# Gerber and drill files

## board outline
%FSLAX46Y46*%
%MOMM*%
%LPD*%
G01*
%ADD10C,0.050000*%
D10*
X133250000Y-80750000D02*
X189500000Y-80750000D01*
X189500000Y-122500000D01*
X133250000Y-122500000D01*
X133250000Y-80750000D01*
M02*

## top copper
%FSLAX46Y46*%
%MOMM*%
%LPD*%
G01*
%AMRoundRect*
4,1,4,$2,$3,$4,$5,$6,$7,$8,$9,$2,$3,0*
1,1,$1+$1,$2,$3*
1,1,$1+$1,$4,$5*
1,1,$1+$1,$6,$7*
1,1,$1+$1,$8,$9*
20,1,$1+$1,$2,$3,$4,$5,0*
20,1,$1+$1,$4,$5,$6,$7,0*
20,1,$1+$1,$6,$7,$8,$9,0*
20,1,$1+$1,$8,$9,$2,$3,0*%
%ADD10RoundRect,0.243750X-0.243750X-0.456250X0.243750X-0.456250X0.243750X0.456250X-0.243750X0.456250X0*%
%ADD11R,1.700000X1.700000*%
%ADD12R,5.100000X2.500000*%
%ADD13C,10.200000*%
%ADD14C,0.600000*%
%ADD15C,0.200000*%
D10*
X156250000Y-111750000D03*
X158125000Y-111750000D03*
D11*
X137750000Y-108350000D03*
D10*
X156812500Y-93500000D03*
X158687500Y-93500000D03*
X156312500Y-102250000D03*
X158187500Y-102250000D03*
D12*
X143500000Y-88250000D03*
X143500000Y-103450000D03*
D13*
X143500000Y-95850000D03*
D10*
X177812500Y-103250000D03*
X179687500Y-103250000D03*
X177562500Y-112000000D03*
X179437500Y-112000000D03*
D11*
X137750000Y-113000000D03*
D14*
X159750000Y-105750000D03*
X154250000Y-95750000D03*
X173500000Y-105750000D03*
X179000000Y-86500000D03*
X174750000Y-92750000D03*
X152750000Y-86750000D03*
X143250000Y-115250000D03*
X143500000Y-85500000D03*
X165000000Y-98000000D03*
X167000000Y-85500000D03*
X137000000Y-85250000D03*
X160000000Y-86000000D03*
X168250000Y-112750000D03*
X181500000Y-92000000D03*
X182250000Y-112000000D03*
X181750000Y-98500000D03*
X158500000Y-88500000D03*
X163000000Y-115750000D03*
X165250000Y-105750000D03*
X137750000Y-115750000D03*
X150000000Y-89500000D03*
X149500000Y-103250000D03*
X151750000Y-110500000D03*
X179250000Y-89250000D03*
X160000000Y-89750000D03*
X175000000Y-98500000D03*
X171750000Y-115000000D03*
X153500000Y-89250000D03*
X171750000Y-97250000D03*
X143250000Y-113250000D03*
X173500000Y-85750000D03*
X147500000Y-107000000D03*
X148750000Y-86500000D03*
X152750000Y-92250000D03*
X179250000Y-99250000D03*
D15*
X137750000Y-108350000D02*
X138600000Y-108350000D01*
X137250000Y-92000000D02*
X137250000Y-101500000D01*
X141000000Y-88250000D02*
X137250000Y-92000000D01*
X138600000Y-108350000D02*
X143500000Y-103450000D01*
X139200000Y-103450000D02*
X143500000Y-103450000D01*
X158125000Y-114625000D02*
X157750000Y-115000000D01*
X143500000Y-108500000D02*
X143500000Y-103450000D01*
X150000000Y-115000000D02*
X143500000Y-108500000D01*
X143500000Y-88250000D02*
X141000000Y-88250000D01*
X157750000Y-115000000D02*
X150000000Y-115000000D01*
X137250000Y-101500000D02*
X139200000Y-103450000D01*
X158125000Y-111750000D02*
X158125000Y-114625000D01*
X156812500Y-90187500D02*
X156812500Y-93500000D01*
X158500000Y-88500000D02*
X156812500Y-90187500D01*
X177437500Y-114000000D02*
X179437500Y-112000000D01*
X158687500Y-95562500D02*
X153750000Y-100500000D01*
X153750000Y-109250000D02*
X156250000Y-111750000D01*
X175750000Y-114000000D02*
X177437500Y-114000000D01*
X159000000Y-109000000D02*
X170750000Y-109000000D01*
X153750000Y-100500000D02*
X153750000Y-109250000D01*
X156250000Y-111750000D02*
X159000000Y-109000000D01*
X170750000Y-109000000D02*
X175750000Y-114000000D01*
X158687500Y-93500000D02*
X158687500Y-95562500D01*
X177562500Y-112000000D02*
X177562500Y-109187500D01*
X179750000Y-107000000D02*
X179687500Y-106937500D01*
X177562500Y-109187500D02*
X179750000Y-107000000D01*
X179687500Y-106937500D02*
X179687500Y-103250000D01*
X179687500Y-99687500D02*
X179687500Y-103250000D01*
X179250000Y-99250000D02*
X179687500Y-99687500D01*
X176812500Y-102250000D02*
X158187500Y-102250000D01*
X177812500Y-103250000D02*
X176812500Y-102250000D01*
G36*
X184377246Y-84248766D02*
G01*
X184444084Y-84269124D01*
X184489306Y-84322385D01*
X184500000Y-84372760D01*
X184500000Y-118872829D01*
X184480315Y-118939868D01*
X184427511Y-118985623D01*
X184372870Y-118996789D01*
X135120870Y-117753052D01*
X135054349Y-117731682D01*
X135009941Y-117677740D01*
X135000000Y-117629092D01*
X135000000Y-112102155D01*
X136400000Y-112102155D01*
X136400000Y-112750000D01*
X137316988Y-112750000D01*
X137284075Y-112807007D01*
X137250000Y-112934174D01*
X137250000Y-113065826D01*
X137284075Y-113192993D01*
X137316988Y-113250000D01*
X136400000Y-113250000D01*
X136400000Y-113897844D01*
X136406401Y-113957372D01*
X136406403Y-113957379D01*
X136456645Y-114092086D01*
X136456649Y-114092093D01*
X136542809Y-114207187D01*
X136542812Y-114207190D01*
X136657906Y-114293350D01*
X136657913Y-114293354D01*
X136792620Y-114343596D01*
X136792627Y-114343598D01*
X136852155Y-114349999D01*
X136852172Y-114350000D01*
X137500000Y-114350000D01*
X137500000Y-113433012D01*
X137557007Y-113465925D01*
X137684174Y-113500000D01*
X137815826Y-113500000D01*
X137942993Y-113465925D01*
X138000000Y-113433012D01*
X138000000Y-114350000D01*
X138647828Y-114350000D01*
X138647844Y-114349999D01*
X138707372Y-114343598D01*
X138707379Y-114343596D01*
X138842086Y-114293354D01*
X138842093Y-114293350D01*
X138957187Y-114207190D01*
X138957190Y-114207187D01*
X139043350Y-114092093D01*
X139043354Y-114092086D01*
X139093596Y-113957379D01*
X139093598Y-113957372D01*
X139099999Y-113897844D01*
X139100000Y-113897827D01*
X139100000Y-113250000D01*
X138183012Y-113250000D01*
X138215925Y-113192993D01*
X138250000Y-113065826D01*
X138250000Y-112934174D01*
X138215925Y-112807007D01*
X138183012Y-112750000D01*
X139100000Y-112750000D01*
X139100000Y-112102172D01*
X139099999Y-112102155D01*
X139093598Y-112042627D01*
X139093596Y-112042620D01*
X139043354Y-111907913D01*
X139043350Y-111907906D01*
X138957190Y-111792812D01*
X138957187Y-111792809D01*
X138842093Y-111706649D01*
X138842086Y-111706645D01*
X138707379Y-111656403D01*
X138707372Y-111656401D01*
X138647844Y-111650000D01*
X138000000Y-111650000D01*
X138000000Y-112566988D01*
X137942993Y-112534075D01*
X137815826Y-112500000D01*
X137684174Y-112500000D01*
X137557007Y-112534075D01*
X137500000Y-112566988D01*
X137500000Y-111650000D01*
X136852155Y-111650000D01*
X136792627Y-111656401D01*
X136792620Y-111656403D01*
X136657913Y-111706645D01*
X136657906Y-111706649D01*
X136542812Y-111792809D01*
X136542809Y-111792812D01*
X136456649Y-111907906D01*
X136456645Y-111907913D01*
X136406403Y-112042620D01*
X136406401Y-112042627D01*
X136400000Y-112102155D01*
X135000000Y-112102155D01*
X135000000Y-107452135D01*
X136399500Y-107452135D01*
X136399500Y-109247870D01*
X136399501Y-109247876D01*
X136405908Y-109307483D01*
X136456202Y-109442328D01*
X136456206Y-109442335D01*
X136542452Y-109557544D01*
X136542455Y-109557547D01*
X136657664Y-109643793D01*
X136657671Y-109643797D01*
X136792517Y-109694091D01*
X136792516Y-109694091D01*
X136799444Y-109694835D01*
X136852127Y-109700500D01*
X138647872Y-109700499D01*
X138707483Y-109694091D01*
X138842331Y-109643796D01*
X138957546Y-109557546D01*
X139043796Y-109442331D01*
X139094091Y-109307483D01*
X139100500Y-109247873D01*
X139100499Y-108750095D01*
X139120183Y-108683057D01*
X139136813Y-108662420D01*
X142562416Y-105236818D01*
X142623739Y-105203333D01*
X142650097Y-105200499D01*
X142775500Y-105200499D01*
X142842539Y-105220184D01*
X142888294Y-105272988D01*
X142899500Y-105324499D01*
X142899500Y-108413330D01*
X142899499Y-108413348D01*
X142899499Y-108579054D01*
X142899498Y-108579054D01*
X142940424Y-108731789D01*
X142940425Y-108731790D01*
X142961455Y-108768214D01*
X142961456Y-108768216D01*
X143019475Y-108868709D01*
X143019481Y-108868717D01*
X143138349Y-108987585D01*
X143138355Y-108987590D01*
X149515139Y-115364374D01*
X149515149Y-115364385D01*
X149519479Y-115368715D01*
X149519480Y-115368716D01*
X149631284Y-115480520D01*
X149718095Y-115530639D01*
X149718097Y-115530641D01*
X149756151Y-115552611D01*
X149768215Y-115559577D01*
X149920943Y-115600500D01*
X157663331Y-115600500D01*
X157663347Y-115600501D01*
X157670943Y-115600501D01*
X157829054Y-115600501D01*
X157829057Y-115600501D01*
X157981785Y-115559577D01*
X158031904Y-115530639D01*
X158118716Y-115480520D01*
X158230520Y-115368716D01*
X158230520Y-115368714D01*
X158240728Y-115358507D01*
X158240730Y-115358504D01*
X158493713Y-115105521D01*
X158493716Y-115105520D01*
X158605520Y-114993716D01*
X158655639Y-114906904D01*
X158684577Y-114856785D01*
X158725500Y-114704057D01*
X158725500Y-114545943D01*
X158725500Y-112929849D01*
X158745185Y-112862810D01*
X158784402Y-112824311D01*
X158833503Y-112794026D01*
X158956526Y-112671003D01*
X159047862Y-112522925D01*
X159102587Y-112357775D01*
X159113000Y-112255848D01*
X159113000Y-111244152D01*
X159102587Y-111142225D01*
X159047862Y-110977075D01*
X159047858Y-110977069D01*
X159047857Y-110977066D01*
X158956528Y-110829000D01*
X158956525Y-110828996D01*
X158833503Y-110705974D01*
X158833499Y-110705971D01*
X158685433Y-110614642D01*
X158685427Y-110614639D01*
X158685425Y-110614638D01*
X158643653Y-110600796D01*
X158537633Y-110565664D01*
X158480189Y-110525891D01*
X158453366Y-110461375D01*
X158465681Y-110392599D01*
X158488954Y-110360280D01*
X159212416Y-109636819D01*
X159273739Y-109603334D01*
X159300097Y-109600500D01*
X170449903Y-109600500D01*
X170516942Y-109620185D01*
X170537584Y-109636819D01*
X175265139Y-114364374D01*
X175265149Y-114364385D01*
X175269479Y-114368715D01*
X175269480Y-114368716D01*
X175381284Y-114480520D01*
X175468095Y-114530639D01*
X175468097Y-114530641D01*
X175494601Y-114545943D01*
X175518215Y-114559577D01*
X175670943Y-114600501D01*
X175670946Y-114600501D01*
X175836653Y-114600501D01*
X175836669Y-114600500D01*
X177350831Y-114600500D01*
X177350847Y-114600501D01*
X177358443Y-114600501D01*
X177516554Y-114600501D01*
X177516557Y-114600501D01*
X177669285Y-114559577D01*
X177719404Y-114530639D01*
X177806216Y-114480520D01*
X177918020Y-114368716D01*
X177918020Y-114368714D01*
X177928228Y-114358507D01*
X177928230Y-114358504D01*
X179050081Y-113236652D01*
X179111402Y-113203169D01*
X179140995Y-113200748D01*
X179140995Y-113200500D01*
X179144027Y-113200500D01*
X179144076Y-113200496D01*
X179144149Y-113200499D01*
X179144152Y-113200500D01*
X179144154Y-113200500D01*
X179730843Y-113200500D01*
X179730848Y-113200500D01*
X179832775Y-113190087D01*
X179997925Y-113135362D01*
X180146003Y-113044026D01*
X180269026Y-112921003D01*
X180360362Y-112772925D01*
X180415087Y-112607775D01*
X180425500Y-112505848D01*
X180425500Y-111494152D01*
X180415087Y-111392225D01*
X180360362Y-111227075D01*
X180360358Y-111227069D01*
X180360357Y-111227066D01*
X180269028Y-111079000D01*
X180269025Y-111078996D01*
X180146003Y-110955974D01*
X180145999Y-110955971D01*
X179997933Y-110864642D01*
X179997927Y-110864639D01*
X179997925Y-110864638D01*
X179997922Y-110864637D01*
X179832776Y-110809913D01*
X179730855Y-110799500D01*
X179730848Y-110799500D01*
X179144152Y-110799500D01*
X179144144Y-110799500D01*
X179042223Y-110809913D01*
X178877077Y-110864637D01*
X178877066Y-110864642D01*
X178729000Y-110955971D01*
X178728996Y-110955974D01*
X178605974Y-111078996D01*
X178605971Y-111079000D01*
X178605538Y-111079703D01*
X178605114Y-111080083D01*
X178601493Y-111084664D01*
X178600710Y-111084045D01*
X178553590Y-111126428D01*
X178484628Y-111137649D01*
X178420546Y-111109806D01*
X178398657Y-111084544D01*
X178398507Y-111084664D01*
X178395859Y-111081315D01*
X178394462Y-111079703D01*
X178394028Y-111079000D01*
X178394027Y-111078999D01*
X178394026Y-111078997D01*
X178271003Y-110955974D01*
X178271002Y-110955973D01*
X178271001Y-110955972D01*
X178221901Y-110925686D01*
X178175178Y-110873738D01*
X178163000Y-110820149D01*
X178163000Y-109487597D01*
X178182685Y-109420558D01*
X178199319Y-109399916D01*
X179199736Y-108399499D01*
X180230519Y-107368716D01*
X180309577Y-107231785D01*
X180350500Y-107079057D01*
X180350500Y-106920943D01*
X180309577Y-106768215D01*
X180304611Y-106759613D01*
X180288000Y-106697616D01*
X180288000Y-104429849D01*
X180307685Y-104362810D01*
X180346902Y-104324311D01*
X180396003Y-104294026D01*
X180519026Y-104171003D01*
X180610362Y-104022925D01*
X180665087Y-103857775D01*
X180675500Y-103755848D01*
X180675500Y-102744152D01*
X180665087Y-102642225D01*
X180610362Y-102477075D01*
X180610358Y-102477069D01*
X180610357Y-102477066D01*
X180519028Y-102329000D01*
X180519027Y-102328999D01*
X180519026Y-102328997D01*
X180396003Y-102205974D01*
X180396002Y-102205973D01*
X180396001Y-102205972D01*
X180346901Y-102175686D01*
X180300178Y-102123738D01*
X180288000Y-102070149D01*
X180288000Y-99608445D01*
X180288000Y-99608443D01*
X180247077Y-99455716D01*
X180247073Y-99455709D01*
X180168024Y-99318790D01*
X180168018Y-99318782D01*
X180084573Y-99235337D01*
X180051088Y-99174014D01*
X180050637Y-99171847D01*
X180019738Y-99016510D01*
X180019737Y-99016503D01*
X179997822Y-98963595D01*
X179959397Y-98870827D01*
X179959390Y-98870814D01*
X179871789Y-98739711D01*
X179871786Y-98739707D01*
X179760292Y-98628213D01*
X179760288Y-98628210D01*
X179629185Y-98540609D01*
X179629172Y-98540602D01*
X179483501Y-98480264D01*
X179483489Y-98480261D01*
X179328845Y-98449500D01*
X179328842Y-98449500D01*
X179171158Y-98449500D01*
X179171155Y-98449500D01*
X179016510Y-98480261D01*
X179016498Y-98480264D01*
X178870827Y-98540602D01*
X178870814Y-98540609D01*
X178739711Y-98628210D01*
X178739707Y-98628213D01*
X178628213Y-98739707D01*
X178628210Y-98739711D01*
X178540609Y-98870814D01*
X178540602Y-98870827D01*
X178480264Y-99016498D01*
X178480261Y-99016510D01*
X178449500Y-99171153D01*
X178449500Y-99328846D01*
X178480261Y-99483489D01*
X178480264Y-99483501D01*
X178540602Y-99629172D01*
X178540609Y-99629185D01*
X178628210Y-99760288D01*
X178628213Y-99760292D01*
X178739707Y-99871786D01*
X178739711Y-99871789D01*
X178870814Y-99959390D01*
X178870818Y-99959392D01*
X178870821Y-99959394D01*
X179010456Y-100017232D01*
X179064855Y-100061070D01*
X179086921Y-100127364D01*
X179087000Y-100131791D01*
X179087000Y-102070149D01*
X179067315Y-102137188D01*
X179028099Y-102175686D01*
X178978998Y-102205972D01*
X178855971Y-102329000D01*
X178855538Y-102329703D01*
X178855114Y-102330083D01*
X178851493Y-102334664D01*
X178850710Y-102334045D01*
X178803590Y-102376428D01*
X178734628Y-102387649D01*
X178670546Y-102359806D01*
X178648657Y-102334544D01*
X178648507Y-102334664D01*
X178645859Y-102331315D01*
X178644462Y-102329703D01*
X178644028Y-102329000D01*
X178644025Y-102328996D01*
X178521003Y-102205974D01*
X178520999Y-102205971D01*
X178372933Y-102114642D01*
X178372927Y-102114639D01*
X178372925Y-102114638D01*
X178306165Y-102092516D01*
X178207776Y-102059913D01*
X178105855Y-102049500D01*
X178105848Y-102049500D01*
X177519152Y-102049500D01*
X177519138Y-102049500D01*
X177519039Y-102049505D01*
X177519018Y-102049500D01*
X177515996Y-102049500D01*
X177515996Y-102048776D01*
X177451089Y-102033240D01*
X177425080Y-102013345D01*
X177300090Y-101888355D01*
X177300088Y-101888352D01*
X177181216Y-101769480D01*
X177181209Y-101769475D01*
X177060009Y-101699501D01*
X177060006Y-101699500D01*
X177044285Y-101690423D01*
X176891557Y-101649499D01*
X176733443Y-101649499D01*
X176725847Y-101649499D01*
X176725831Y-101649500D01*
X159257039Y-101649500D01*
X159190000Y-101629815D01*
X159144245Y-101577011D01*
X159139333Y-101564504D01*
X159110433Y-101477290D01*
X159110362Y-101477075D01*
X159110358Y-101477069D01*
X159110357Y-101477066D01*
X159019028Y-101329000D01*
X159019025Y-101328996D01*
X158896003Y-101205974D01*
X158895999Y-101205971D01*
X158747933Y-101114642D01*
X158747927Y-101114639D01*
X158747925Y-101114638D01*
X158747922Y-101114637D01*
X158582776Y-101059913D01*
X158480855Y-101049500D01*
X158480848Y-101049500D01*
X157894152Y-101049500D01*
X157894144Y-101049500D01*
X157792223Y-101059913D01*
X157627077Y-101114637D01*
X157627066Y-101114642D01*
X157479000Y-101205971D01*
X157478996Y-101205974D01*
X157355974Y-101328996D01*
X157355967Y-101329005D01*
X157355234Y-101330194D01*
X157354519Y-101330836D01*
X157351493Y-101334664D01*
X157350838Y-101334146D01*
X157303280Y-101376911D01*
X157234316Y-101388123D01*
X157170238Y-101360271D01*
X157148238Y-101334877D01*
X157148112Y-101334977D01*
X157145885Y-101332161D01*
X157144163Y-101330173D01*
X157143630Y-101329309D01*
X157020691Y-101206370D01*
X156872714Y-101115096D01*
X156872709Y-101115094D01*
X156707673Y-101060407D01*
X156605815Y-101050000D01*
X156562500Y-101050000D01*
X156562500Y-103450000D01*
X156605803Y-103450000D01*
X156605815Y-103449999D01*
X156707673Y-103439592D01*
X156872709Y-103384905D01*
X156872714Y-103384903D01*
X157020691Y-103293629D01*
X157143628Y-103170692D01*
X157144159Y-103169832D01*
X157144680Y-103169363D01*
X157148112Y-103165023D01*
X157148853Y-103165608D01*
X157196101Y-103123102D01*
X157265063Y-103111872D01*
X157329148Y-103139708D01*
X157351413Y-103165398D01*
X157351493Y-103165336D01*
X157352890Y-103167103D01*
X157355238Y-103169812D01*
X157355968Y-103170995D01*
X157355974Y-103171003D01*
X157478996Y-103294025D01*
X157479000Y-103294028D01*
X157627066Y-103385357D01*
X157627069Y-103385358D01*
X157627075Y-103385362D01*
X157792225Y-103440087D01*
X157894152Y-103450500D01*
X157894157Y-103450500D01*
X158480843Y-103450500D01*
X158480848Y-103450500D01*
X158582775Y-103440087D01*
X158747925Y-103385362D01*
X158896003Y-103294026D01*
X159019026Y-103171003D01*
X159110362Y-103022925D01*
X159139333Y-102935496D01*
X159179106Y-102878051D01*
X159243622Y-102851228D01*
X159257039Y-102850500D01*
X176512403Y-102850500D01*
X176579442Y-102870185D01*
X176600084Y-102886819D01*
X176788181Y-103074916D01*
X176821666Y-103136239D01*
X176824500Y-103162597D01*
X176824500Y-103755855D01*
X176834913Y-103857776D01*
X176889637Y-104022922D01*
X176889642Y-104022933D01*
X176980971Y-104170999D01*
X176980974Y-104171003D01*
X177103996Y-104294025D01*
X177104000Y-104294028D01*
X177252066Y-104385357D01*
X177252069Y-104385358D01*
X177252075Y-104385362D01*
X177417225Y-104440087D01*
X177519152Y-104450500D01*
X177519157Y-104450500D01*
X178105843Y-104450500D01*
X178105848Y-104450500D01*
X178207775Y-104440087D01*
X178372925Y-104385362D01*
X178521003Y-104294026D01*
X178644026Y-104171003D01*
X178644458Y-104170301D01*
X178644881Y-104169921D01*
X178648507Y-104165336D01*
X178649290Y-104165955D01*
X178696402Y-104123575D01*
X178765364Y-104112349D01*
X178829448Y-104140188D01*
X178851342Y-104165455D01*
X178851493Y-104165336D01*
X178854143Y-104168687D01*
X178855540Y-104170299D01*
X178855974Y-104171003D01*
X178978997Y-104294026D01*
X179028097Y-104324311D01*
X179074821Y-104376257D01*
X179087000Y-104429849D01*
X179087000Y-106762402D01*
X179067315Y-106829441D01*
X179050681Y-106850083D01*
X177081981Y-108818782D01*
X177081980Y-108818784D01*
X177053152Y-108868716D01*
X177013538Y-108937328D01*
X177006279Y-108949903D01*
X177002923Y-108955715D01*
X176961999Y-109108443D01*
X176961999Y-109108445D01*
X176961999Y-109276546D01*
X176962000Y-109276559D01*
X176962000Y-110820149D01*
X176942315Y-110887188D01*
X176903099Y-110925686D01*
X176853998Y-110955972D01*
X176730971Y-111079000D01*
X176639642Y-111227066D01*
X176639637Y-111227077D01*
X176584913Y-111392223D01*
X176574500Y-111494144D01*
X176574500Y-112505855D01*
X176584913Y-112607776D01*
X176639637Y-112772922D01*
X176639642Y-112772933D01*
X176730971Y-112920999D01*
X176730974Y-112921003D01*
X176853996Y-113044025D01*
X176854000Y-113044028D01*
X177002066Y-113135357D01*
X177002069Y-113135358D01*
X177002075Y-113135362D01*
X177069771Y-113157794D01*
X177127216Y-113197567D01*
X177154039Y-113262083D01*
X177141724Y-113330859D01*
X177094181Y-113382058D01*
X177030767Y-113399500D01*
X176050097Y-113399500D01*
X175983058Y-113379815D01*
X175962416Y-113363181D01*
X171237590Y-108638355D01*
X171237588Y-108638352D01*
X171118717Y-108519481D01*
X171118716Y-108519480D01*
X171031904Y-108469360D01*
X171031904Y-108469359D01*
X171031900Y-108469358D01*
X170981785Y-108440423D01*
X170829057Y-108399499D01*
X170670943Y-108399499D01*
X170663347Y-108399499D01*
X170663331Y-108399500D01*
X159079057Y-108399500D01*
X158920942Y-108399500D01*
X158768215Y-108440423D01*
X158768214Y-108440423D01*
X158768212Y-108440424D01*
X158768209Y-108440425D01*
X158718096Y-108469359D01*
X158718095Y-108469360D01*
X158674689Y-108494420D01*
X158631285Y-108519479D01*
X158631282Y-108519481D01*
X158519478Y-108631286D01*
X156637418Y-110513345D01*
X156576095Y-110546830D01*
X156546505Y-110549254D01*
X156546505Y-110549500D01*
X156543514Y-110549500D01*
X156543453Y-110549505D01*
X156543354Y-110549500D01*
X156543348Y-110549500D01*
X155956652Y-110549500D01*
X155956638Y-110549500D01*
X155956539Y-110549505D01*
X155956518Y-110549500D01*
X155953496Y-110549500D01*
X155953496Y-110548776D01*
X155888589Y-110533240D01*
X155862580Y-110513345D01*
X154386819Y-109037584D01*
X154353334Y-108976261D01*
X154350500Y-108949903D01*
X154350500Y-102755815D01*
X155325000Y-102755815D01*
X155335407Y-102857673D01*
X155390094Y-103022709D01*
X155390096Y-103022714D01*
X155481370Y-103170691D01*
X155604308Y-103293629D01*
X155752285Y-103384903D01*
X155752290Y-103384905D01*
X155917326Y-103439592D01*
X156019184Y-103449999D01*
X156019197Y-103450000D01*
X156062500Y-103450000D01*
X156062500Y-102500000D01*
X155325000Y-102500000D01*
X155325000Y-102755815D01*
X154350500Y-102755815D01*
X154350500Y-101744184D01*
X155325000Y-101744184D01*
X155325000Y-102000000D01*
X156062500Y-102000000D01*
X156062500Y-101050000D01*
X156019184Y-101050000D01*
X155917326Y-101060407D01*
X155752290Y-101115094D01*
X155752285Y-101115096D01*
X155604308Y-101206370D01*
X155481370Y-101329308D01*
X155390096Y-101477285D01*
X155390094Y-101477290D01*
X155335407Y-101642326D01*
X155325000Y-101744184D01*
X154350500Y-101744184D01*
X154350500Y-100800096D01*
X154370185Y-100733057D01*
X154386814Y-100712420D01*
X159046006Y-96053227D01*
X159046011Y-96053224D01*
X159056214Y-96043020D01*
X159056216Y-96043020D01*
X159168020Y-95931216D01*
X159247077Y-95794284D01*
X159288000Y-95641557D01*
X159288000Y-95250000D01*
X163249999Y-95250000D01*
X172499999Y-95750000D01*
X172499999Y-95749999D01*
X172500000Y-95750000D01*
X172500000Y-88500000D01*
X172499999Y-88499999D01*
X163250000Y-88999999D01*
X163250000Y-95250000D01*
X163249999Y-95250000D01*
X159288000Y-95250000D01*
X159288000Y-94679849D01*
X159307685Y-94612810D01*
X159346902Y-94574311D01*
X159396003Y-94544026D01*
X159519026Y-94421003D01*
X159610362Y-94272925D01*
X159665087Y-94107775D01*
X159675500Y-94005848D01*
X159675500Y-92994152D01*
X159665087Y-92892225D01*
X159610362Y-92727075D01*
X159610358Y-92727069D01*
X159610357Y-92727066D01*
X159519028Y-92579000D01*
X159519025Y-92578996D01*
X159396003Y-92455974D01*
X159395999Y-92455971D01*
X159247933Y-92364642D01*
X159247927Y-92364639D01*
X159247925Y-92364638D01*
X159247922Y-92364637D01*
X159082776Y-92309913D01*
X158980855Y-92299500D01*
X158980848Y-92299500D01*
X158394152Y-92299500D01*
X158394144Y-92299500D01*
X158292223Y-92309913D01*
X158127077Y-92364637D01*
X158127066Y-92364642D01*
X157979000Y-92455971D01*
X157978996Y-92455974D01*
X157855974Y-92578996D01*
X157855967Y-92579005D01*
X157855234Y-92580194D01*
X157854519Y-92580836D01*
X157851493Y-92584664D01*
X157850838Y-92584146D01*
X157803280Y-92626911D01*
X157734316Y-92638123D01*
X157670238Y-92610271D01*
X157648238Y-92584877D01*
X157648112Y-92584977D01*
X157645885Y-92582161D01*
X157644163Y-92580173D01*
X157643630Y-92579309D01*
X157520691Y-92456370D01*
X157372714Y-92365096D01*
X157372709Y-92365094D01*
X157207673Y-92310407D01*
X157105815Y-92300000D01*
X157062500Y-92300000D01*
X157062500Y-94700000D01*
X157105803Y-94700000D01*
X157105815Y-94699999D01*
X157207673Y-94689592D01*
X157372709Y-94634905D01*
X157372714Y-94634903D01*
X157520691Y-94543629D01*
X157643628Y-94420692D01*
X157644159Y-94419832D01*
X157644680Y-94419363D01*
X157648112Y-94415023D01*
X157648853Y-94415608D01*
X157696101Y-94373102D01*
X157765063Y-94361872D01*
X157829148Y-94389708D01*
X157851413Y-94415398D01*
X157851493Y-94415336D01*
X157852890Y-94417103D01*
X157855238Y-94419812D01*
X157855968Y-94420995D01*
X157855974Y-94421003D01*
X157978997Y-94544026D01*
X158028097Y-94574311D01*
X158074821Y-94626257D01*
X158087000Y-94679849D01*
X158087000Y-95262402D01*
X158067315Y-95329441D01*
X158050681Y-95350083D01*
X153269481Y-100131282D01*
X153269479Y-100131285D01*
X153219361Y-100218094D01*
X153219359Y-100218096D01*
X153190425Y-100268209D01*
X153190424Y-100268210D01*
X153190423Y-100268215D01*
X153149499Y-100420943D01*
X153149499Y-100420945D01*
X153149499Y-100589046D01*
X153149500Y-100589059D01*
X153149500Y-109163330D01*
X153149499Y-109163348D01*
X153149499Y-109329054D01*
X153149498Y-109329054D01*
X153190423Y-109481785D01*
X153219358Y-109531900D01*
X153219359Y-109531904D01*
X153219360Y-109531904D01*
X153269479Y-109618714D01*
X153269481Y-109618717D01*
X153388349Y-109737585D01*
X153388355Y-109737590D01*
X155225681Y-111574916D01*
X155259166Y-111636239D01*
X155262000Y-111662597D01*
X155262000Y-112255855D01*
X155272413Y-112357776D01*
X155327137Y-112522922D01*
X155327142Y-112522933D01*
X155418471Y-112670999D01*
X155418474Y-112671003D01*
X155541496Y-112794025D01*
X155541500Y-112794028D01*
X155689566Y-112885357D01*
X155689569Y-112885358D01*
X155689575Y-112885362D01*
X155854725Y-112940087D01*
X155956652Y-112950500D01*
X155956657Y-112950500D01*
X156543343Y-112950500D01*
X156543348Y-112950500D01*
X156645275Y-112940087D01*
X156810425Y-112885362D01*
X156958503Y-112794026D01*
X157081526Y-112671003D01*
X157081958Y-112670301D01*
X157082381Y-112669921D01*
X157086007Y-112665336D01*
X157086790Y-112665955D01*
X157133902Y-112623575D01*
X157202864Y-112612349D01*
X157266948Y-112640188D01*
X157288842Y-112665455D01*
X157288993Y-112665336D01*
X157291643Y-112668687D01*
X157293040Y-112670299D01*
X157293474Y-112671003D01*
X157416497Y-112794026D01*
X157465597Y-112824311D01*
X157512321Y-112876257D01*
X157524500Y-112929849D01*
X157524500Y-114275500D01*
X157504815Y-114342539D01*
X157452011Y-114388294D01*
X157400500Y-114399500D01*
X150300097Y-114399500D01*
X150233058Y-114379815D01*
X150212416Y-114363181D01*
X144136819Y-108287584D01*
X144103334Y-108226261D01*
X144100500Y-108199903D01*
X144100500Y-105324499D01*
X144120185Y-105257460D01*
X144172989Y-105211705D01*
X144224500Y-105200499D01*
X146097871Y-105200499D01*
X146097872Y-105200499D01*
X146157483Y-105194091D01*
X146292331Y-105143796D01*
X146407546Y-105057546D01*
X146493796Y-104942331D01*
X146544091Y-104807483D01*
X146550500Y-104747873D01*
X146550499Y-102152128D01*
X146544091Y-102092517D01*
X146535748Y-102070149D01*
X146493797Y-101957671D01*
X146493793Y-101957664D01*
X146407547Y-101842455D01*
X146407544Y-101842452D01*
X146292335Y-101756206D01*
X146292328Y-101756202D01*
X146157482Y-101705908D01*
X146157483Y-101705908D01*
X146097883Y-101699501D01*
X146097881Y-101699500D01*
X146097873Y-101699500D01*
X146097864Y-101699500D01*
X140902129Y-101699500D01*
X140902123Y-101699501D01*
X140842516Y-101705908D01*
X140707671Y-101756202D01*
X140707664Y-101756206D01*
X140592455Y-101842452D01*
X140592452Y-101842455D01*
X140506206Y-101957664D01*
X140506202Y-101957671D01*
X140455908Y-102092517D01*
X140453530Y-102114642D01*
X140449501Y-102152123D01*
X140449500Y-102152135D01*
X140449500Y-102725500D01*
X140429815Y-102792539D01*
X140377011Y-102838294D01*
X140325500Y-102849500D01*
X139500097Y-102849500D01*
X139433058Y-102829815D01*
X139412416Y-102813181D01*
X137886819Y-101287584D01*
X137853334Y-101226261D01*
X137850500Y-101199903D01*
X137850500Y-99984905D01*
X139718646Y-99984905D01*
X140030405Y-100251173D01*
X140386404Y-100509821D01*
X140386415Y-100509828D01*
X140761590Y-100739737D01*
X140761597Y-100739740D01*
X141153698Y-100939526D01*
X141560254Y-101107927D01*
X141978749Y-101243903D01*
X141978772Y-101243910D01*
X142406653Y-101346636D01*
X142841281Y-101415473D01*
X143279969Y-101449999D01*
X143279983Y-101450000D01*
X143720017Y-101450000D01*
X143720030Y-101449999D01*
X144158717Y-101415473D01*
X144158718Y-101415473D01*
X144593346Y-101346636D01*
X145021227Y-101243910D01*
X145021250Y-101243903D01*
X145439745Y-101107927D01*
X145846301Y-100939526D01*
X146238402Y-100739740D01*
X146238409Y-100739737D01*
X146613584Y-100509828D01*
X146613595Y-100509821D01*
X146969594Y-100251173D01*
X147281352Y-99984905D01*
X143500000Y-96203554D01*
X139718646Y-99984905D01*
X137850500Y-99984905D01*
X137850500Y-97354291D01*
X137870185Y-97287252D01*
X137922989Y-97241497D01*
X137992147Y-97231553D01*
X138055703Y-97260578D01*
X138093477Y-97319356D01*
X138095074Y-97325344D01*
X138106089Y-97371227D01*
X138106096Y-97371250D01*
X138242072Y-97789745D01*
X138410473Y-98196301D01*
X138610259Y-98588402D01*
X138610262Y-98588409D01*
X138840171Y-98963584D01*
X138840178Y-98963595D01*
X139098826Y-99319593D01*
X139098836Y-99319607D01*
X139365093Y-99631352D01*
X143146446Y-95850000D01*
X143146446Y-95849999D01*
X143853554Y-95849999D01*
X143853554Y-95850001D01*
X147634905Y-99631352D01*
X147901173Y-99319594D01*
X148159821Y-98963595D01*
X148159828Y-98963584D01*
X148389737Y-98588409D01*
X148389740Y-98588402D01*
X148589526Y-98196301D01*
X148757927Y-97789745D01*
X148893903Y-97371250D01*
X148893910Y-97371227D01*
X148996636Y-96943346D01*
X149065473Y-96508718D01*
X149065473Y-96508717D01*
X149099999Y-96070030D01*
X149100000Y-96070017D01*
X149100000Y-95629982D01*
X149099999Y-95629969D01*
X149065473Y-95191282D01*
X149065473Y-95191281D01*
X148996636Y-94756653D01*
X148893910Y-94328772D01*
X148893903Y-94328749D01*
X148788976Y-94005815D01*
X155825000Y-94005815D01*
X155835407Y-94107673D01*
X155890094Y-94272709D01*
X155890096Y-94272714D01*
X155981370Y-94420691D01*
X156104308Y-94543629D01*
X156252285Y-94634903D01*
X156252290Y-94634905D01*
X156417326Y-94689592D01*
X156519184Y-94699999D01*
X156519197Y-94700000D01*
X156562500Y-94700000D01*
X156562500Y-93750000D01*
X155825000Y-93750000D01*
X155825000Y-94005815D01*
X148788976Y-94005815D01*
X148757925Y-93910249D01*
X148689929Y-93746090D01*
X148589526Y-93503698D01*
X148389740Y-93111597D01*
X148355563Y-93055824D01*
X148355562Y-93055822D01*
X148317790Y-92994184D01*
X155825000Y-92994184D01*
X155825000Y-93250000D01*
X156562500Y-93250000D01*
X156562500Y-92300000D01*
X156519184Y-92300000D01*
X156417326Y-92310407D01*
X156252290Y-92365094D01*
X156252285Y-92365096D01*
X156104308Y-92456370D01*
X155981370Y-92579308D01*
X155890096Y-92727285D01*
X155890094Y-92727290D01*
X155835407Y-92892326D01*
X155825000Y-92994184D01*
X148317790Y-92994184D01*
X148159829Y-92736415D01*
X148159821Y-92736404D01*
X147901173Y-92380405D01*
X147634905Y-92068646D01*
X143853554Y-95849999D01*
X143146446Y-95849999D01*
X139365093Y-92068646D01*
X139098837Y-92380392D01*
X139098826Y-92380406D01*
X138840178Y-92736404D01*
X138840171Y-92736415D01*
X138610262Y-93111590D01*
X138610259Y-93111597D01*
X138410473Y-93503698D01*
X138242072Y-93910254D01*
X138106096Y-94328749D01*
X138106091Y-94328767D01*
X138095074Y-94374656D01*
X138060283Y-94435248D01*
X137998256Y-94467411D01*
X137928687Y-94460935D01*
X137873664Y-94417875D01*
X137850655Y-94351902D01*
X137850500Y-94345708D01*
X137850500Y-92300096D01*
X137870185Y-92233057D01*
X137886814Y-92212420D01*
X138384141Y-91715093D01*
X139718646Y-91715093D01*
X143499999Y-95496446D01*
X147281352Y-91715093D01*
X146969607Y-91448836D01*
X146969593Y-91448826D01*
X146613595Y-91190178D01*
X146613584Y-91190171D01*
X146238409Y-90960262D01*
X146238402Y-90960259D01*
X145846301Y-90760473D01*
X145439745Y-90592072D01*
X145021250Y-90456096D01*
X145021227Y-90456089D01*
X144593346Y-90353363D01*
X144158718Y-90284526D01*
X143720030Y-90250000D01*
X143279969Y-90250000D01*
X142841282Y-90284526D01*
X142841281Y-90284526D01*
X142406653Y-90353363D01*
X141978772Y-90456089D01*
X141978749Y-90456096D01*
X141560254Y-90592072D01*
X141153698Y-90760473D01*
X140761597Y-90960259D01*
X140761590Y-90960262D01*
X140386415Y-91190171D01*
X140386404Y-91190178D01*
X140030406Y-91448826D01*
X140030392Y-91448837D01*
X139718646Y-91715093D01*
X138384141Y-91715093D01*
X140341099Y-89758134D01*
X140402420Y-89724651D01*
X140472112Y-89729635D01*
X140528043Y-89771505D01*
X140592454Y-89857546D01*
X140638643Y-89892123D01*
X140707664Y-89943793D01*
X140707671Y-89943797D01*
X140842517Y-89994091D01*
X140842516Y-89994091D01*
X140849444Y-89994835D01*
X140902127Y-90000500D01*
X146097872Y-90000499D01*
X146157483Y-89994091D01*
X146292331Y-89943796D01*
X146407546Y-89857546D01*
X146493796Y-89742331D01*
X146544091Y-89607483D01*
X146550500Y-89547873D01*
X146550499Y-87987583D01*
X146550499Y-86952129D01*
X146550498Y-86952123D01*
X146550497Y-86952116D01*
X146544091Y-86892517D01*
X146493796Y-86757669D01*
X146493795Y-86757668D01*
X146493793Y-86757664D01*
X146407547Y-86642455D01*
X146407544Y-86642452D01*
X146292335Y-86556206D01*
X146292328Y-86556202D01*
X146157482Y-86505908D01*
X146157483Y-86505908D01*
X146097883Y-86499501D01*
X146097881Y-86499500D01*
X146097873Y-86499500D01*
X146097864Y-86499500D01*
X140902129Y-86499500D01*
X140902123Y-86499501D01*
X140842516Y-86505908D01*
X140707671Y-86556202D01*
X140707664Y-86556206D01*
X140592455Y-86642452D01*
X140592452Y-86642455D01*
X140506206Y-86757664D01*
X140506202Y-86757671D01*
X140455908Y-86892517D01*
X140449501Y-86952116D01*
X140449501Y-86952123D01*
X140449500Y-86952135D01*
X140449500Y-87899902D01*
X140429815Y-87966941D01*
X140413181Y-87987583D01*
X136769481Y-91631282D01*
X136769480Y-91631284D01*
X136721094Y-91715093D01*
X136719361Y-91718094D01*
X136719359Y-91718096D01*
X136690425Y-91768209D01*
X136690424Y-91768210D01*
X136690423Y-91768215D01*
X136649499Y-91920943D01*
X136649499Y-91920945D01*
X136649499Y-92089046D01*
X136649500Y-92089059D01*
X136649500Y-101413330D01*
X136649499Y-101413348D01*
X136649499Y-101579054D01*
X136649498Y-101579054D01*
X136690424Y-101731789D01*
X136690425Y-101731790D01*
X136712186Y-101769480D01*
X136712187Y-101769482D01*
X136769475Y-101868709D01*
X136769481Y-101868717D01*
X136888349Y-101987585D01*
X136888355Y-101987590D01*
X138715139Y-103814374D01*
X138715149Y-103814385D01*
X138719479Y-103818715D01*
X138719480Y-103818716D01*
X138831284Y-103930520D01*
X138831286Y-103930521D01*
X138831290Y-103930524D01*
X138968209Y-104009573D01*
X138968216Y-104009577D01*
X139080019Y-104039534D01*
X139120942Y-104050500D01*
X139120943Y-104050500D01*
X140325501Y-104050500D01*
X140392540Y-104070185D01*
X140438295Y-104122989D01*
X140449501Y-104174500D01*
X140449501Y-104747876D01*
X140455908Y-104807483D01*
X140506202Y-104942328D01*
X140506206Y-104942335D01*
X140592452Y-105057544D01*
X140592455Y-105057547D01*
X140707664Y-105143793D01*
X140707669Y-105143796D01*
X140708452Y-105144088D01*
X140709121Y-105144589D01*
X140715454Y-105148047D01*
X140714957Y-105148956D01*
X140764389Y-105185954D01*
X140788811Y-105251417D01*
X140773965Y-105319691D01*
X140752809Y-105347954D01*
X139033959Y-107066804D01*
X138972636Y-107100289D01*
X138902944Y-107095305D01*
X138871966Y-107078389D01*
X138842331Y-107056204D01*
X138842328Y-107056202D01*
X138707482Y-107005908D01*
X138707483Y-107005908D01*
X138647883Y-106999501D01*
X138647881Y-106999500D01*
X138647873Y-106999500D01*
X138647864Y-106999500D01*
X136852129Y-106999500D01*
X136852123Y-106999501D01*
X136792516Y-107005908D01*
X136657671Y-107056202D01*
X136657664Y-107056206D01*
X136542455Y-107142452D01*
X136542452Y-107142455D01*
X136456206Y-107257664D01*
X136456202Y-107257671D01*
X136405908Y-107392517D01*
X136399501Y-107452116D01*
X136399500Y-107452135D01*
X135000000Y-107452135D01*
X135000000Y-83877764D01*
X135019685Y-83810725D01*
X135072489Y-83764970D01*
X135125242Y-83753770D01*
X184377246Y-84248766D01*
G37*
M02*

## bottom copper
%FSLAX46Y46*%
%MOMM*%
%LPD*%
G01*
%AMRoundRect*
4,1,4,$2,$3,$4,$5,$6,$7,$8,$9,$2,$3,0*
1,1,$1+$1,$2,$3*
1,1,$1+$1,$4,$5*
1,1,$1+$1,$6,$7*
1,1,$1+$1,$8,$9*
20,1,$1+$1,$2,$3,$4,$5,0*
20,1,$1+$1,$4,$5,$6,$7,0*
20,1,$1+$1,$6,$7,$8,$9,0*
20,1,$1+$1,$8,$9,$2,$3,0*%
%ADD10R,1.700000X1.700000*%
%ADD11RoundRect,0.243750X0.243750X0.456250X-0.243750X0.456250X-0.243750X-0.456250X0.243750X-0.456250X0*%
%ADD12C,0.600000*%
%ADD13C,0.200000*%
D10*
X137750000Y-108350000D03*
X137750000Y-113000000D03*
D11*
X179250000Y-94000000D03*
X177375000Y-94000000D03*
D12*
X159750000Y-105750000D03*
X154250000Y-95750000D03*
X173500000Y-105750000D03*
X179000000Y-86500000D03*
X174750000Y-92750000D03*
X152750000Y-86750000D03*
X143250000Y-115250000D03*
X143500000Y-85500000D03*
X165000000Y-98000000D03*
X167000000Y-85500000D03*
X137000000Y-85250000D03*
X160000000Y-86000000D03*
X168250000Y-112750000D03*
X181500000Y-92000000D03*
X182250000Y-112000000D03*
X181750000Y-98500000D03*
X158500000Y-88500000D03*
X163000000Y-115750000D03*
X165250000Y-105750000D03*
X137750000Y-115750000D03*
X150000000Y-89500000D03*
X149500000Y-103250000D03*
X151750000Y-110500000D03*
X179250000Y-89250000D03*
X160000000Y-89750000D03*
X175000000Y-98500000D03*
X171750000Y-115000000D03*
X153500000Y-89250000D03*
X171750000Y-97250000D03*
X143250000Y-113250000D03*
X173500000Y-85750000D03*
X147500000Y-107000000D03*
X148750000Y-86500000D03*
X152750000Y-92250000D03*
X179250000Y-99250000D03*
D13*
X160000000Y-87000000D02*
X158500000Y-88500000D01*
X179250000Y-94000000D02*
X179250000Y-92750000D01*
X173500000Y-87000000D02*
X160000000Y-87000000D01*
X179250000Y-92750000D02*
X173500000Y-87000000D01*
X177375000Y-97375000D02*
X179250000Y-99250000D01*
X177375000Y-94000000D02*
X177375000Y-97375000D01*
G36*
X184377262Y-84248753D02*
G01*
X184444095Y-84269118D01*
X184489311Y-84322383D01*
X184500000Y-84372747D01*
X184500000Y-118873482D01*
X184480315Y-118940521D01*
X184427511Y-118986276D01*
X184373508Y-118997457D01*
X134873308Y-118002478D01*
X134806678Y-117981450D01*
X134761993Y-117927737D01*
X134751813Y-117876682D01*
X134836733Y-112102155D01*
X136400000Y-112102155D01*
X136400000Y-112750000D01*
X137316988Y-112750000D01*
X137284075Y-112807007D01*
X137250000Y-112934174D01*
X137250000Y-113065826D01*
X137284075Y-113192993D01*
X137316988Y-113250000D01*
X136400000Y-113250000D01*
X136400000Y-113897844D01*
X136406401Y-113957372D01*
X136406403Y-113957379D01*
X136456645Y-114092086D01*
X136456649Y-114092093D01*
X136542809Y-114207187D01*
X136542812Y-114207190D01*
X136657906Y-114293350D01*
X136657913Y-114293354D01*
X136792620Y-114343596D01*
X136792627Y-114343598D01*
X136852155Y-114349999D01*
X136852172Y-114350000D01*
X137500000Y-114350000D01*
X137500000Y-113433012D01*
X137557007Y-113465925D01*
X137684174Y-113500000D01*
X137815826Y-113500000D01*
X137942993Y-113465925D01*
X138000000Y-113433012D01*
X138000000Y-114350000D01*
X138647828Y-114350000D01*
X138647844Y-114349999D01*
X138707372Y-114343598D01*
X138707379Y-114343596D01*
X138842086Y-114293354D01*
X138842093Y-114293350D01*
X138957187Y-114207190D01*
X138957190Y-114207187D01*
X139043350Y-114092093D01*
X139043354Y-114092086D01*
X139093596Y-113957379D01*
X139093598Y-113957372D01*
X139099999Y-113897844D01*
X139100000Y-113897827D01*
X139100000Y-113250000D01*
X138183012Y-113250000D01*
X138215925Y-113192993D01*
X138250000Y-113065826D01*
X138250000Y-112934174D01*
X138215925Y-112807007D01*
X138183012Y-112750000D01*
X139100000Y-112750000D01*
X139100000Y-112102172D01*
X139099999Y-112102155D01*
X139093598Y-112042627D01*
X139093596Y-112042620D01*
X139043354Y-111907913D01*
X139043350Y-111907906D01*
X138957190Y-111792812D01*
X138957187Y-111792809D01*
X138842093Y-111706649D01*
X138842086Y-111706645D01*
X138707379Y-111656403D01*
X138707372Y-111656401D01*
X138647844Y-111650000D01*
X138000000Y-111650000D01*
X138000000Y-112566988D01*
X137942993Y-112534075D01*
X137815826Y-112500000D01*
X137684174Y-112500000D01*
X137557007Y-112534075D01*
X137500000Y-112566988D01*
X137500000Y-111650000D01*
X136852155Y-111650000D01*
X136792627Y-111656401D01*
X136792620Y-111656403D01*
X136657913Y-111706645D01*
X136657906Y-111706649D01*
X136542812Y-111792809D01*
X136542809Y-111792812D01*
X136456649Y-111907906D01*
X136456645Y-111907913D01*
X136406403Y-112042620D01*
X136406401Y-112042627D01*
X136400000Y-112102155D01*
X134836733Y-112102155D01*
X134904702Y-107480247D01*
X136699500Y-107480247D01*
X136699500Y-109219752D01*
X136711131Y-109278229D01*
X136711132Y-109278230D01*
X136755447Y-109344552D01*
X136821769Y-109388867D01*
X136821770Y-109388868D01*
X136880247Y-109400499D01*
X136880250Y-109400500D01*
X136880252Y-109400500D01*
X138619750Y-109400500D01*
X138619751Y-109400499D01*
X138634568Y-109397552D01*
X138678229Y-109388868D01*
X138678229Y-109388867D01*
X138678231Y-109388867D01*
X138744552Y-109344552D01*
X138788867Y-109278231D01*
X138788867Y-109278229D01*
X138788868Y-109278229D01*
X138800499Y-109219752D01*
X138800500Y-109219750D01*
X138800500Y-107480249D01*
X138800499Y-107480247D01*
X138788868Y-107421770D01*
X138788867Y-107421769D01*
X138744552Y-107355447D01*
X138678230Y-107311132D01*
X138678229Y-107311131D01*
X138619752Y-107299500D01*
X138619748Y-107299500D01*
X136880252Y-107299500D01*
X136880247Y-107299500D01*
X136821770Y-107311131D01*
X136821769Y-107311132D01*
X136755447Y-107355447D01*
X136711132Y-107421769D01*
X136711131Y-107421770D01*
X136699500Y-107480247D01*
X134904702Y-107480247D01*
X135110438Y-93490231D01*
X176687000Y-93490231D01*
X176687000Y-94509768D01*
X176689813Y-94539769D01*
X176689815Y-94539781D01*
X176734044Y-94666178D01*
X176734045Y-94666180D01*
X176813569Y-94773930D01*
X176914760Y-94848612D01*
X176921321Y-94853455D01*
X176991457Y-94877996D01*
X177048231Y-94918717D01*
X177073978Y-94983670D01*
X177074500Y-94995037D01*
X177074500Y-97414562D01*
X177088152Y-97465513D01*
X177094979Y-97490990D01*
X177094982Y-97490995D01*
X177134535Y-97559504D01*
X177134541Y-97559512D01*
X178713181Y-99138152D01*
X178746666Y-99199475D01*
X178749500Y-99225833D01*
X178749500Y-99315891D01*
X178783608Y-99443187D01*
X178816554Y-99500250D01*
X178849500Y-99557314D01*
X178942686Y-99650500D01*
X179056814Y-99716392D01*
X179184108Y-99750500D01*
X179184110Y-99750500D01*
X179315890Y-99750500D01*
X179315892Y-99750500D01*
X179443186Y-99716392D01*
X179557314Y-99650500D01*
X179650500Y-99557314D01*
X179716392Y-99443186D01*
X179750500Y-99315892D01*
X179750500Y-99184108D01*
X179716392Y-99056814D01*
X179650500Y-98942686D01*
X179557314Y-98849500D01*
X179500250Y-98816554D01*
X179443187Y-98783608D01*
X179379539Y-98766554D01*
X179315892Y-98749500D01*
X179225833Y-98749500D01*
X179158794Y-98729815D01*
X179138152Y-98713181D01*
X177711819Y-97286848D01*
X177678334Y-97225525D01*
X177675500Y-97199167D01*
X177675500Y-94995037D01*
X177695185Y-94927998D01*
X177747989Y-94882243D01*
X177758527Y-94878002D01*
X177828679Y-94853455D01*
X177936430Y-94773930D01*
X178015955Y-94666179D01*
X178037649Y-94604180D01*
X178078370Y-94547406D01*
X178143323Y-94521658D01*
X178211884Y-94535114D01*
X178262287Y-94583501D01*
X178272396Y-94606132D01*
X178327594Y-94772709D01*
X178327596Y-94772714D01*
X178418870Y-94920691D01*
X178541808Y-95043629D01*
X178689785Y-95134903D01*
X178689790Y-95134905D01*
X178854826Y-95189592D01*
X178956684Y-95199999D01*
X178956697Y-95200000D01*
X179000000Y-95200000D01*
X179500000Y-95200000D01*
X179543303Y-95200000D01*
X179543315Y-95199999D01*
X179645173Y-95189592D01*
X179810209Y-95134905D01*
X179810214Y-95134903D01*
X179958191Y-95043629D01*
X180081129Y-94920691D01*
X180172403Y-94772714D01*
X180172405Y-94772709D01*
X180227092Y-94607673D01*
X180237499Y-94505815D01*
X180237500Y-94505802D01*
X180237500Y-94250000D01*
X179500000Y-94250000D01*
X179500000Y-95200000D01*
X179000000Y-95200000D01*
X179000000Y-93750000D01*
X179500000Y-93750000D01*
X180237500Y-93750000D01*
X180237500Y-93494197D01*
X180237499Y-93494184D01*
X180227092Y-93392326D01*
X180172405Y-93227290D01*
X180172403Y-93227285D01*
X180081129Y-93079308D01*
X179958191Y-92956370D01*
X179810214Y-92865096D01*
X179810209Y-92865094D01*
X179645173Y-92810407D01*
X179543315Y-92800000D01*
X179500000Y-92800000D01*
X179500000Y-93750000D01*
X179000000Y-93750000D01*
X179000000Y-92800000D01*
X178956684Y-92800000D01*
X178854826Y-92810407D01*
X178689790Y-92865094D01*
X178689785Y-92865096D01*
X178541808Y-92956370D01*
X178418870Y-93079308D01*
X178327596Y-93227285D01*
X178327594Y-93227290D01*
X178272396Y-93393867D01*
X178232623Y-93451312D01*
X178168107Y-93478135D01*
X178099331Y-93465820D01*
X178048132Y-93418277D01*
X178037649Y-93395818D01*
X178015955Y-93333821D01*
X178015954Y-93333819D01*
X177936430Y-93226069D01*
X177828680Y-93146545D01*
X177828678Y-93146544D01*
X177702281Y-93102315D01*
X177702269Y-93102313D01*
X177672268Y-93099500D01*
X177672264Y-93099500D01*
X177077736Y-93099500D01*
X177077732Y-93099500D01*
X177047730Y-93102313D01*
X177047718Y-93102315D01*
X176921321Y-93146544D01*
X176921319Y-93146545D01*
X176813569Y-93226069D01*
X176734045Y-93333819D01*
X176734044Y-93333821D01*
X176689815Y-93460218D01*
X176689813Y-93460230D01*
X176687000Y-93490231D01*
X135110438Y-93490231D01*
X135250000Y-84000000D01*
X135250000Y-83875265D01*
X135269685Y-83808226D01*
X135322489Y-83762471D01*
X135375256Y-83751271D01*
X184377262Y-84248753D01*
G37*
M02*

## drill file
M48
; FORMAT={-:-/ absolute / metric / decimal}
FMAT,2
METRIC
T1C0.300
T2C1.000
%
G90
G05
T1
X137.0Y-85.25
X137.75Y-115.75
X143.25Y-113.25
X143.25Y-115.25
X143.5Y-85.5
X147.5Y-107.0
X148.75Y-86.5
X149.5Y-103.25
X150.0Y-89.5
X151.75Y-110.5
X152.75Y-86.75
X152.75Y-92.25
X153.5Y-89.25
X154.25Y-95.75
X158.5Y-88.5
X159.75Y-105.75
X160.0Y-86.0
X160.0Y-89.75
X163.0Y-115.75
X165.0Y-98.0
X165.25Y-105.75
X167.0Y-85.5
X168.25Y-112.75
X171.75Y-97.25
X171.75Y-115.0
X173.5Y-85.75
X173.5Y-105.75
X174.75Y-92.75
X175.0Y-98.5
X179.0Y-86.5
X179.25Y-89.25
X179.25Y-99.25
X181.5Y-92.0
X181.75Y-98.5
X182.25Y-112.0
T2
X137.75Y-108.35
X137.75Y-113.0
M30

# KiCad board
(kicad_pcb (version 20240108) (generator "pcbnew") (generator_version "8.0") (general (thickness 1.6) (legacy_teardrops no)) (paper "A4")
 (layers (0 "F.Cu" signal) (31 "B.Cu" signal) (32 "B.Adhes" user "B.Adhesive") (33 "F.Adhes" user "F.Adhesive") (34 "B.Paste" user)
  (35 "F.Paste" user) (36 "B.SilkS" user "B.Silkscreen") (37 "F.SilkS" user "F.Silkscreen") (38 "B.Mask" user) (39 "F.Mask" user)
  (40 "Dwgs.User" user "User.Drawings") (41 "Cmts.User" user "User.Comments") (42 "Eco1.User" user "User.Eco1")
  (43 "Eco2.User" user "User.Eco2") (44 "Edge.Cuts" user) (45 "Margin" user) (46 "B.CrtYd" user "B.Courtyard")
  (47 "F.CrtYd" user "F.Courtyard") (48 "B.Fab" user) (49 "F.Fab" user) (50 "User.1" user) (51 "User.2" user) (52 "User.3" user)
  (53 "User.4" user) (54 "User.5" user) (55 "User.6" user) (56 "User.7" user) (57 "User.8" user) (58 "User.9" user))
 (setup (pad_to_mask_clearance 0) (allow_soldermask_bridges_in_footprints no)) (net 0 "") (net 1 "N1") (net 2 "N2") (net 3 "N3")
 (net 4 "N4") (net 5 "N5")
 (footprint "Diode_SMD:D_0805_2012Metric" (layer "F.Cu") (at 157.1875 111.75)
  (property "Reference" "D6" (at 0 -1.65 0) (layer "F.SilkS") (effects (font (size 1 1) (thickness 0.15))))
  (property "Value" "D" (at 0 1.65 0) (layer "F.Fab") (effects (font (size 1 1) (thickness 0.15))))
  (pad "1" smd roundrect (at -0.9375 0) (size 0.975 1.4) (layers "F.Cu" "F.Paste" "F.Mask") (roundrect_rratio 0.25) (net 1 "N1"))
  (pad "2" smd roundrect (at 0.9375 0) (size 0.975 1.4) (layers "F.Cu" "F.Paste" "F.Mask") (roundrect_rratio 0.25) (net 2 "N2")))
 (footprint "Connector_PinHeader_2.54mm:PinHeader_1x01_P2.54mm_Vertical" (layer "F.Cu") (at 137.75 108.35)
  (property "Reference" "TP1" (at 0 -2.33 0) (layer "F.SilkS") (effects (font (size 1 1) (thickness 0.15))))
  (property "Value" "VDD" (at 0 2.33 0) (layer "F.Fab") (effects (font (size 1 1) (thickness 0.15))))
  (pad "1" thru_hole rect (at 0 0) (size 1.7 1.7) (drill 1) (layers "*.Cu" "*.Mask") (remove_unused_layers no) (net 2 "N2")))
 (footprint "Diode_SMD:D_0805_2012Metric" (layer "F.Cu") (at 157.75 93.5)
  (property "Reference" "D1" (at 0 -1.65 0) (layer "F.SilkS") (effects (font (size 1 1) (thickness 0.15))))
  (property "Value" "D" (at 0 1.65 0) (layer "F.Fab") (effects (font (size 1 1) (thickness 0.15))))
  (pad "1" smd roundrect (at -0.9375 0) (size 0.975 1.4) (layers "F.Cu" "F.Paste" "F.Mask") (roundrect_rratio 0.25) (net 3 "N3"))
  (pad "2" smd roundrect (at 0.9375 0) (size 0.975 1.4) (layers "F.Cu" "F.Paste" "F.Mask") (roundrect_rratio 0.25) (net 1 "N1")))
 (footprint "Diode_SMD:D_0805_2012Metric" (layer "F.Cu") (at 157.25 102.25)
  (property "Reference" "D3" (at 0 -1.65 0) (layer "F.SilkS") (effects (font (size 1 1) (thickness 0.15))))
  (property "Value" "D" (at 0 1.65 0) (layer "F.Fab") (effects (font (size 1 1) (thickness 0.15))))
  (pad "1" smd roundrect (at -0.9375 0) (size 0.975 1.4) (layers "F.Cu" "F.Paste" "F.Mask") (roundrect_rratio 0.25) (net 3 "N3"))
  (pad "2" smd roundrect (at 0.9375 0) (size 0.975 1.4) (layers "F.Cu" "F.Paste" "F.Mask") (roundrect_rratio 0.25) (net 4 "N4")))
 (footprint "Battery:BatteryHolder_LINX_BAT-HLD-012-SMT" (layer "F.Cu") (at 143.5 95.85 -90)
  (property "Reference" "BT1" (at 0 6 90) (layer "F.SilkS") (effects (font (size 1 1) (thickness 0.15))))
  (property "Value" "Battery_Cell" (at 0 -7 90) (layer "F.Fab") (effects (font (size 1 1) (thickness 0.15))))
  (pad "1" smd rect (at -7.6 0 270) (size 2.5 5.1) (layers "F.Cu" "F.Paste" "F.Mask") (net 2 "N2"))
  (pad "1" smd rect (at 7.6 0 270) (size 2.5 5.1) (layers "F.Cu" "F.Paste" "F.Mask") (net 2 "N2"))
  (pad "2" smd circle (at 0 0 270) (size 10.2 10.2) (layers "F.Cu" "F.Mask") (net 3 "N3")))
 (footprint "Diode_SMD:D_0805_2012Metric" (layer "F.Cu") (at 178.75 103.25)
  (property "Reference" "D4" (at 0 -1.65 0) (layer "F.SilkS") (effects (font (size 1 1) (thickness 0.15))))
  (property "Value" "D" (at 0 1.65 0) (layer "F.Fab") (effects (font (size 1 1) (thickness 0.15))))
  (pad "1" smd roundrect (at -0.9375 0) (size 0.975 1.4) (layers "F.Cu" "F.Paste" "F.Mask") (roundrect_rratio 0.25) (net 4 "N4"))
  (pad "2" smd roundrect (at 0.9375 0) (size 0.975 1.4) (layers "F.Cu" "F.Paste" "F.Mask") (roundrect_rratio 0.25) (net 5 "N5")))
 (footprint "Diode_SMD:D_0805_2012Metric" (layer "F.Cu") (at 178.5 112)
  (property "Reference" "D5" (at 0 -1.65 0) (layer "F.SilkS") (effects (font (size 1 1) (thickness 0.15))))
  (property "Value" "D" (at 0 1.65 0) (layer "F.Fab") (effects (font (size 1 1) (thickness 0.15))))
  (pad "1" smd roundrect (at -0.9375 0) (size 0.975 1.4) (layers "F.Cu" "F.Paste" "F.Mask") (roundrect_rratio 0.25) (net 5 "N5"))
  (pad "2" smd roundrect (at 0.9375 0) (size 0.975 1.4) (layers "F.Cu" "F.Paste" "F.Mask") (roundrect_rratio 0.25) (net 1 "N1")))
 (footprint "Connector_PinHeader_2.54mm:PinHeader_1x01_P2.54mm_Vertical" (layer "F.Cu") (at 137.75 113)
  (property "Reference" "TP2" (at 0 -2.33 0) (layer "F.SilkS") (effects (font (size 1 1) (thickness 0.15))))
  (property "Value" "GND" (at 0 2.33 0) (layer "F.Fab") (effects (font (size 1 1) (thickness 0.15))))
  (pad "1" thru_hole rect (at 0 0) (size 1.7 1.7) (drill 1) (layers "*.Cu" "*.Mask") (remove_unused_layers no) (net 3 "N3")))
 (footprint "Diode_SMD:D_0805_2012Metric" (layer "B.Cu") (at 178.3125 94 180)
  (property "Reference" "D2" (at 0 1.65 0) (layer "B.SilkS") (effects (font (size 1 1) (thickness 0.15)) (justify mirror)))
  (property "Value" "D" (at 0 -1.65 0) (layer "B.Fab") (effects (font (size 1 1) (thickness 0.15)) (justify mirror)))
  (pad "1" smd roundrect (at -0.9375 0 180) (size 0.975 1.4) (layers "B.Cu" "B.Paste" "B.Mask") (roundrect_rratio 0.25) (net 3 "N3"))
  (pad "2" smd roundrect (at 0.9375 0 180) (size 0.975 1.4) (layers "B.Cu" "B.Paste" "B.Mask") (roundrect_rratio 0.25) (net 5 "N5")))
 (gr_rect (start 133.25 80.75) (end 189.5 122.5) (stroke (width 0.05) (type default)) (fill none) (layer "Edge.Cuts"))
 (segment (start 137.75 108.35) (end 138.6 108.35) (width 0.2) (layer "F.Cu") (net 2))
 (segment (start 137.25 92) (end 137.25 101.5) (width 0.2) (layer "F.Cu") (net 2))
 (segment (start 141 88.25) (end 137.25 92) (width 0.2) (layer "F.Cu") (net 2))
 (segment (start 138.6 108.35) (end 143.5 103.45) (width 0.2) (layer "F.Cu") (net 2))
 (segment (start 139.2 103.45) (end 143.5 103.45) (width 0.2) (layer "F.Cu") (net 2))
 (segment (start 158.125 114.625) (end 157.75 115) (width 0.2) (layer "F.Cu") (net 2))
 (segment (start 143.5 108.5) (end 143.5 103.45) (width 0.2) (layer "F.Cu") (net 2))
 (segment (start 150 115) (end 143.5 108.5) (width 0.2) (layer "F.Cu") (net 2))
 (segment (start 143.5 88.25) (end 141 88.25) (width 0.2) (layer "F.Cu") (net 2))
 (segment (start 157.75 115) (end 150 115) (width 0.2) (layer "F.Cu") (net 2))
 (segment (start 137.25 101.5) (end 139.2 103.45) (width 0.2) (layer "F.Cu") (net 2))
 (segment (start 158.125 111.75) (end 158.125 114.625) (width 0.2) (layer "F.Cu") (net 2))
 (segment (start 156.8125 90.1875) (end 156.8125 93.5) (width 0.2) (layer "F.Cu") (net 3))
 (segment (start 158.5 88.5) (end 156.8125 90.1875) (width 0.2) (layer "F.Cu") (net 3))
 (via (at 159.75 105.75) (size 0.6) (drill 0.3) (layers "F.Cu" "B.Cu") (free yes) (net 3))
 (via (at 154.25 95.75) (size 0.6) (drill 0.3) (layers "F.Cu" "B.Cu") (free yes) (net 3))
 (via (at 173.5 105.75) (size 0.6) (drill 0.3) (layers "F.Cu" "B.Cu") (free yes) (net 3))
 (via (at 179 86.5) (size 0.6) (drill 0.3) (layers "F.Cu" "B.Cu") (free yes) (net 3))
 (via (at 174.75 92.75) (size 0.6) (drill 0.3) (layers "F.Cu" "B.Cu") (free yes) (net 3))
 (via (at 152.75 86.75) (size 0.6) (drill 0.3) (layers "F.Cu" "B.Cu") (free yes) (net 3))
 (via (at 143.25 115.25) (size 0.6) (drill 0.3) (layers "F.Cu" "B.Cu") (free yes) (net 3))
 (via (at 143.5 85.5) (size 0.6) (drill 0.3) (layers "F.Cu" "B.Cu") (free yes) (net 3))
 (via (at 165 98) (size 0.6) (drill 0.3) (layers "F.Cu" "B.Cu") (free yes) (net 3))
 (via (at 167 85.5) (size 0.6) (drill 0.3) (layers "F.Cu" "B.Cu") (free yes) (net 3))
 (via (at 137 85.25) (size 0.6) (drill 0.3) (layers "F.Cu" "B.Cu") (free yes) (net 3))
 (via (at 160 86) (size 0.6) (drill 0.3) (layers "F.Cu" "B.Cu") (free yes) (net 3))
 (via (at 168.25 112.75) (size 0.6) (drill 0.3) (layers "F.Cu" "B.Cu") (free yes) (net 3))
 (via (at 181.5 92) (size 0.6) (drill 0.3) (layers "F.Cu" "B.Cu") (free yes) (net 3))
 (via (at 182.25 112) (size 0.6) (drill 0.3) (layers "F.Cu" "B.Cu") (free yes) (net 3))
 (via (at 181.75 98.5) (size 0.6) (drill 0.3) (layers "F.Cu" "B.Cu") (free yes) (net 3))
 (via (at 158.5 88.5) (size 0.6) (drill 0.3) (layers "F.Cu" "B.Cu") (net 3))
 (via (at 163 115.75) (size 0.6) (drill 0.3) (layers "F.Cu" "B.Cu") (free yes) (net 3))
 (via (at 165.25 105.75) (size 0.6) (drill 0.3) (layers "F.Cu" "B.Cu") (free yes) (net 3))
 (via (at 137.75 115.75) (size 0.6) (drill 0.3) (layers "F.Cu" "B.Cu") (free yes) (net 3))
 (via (at 150 89.5) (size 0.6) (drill 0.3) (layers "F.Cu" "B.Cu") (free yes) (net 3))
 (via (at 149.5 103.25) (size 0.6) (drill 0.3) (layers "F.Cu" "B.Cu") (free yes) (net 3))
 (via (at 151.75 110.5) (size 0.6) (drill 0.3) (layers "F.Cu" "B.Cu") (free yes) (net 3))
 (via (at 179.25 89.25) (size 0.6) (drill 0.3) (layers "F.Cu" "B.Cu") (free yes) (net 3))
 (via (at 160 89.75) (size 0.6) (drill 0.3) (layers "F.Cu" "B.Cu") (free yes) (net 3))
 (via (at 175 98.5) (size 0.6) (drill 0.3) (layers "F.Cu" "B.Cu") (free yes) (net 3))
 (via (at 171.75 115) (size 0.6) (drill 0.3) (layers "F.Cu" "B.Cu") (free yes) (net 3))
 (via (at 153.5 89.25) (size 0.6) (drill 0.3) (layers "F.Cu" "B.Cu") (free yes) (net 3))
 (via (at 171.75 97.25) (size 0.6) (drill 0.3) (layers "F.Cu" "B.Cu") (free yes) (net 3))
 (via (at 143.25 113.25) (size 0.6) (drill 0.3) (layers "F.Cu" "B.Cu") (free yes) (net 3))
 (via (at 173.5 85.75) (size 0.6) (drill 0.3) (layers "F.Cu" "B.Cu") (free yes) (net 3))
 (via (at 147.5 107) (size 0.6) (drill 0.3) (layers "F.Cu" "B.Cu") (free yes) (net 3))
 (via (at 148.75 86.5) (size 0.6) (drill 0.3) (layers "F.Cu" "B.Cu") (free yes) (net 3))
 (via (at 152.75 92.25) (size 0.6) (drill 0.3) (layers "F.Cu" "B.Cu") (free yes) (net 3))
 (segment (start 160 87) (end 158.5 88.5) (width 0.2) (layer "B.Cu") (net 3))
 (segment (start 179.25 94) (end 179.25 92.75) (width 0.2) (layer "B.Cu") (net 3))
 (segment (start 173.5 87) (end 160 87) (width 0.2) (layer "B.Cu") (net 3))
 (segment (start 179.25 92.75) (end 173.5 87) (width 0.2) (layer "B.Cu") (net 3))
 (segment (start 177.4375 114) (end 179.4375 112) (width 0.2) (layer "F.Cu") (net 1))
 (segment (start 158.6875 95.5625) (end 153.75 100.5) (width 0.2) (layer "F.Cu") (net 1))
 (segment (start 153.75 109.25) (end 156.25 111.75) (width 0.2) (layer "F.Cu") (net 1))
 (segment (start 175.75 114) (end 177.4375 114) (width 0.2) (layer "F.Cu") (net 1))
 (segment (start 159 109) (end 170.75 109) (width 0.2) (layer "F.Cu") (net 1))
 (segment (start 153.75 100.5) (end 153.75 109.25) (width 0.2) (layer "F.Cu") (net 1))
 (segment (start 156.25 111.75) (end 159 109) (width 0.2) (layer "F.Cu") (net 1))
 (segment (start 170.75 109) (end 175.75 114) (width 0.2) (layer "F.Cu") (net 1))
 (segment (start 158.6875 93.5) (end 158.6875 95.5625) (width 0.2) (layer "F.Cu") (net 1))
 (segment (start 177.5625 112) (end 177.5625 109.1875) (width 0.2) (layer "F.Cu") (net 5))
 (segment (start 179.75 107) (end 179.6875 106.9375) (width 0.2) (layer "F.Cu") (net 5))
 (segment (start 177.5625 109.1875) (end 179.75 107) (width 0.2) (layer "F.Cu") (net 5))
 (segment (start 179.6875 106.9375) (end 179.6875 103.25) (width 0.2) (layer "F.Cu") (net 5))
 (segment (start 179.6875 99.6875) (end 179.6875 103.25) (width 0.2) (layer "F.Cu") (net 5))
 (segment (start 179.25 99.25) (end 179.6875 99.6875) (width 0.2) (layer "F.Cu") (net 5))
 (via (at 179.25 99.25) (size 0.6) (drill 0.3) (layers "F.Cu" "B.Cu") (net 5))
 (segment (start 177.375 97.375) (end 179.25 99.25) (width 0.2) (layer "B.Cu") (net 5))
 (segment (start 177.375 94) (end 177.375 97.375) (width 0.2) (layer "B.Cu") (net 5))
 (segment (start 176.8125 102.25) (end 158.1875 102.25) (width 0.2) (layer "F.Cu") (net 4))
 (segment (start 177.8125 103.25) (end 176.8125 102.25) (width 0.2) (layer "F.Cu") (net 4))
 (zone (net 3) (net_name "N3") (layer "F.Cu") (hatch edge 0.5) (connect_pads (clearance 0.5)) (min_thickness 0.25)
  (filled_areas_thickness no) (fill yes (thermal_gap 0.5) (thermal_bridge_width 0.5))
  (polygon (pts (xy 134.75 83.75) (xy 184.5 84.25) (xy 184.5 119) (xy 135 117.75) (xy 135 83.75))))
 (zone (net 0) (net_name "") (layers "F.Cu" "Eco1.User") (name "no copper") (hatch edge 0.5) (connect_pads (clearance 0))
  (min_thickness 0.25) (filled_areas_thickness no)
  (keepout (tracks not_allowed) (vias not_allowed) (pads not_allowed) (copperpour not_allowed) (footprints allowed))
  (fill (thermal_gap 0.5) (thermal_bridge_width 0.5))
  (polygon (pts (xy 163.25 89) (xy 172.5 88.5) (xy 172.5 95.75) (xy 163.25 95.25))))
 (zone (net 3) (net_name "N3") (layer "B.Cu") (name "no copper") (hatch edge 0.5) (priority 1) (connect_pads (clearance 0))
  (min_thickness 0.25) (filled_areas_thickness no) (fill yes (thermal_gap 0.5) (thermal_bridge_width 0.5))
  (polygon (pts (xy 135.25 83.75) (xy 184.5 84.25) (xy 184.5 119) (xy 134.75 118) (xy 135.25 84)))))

